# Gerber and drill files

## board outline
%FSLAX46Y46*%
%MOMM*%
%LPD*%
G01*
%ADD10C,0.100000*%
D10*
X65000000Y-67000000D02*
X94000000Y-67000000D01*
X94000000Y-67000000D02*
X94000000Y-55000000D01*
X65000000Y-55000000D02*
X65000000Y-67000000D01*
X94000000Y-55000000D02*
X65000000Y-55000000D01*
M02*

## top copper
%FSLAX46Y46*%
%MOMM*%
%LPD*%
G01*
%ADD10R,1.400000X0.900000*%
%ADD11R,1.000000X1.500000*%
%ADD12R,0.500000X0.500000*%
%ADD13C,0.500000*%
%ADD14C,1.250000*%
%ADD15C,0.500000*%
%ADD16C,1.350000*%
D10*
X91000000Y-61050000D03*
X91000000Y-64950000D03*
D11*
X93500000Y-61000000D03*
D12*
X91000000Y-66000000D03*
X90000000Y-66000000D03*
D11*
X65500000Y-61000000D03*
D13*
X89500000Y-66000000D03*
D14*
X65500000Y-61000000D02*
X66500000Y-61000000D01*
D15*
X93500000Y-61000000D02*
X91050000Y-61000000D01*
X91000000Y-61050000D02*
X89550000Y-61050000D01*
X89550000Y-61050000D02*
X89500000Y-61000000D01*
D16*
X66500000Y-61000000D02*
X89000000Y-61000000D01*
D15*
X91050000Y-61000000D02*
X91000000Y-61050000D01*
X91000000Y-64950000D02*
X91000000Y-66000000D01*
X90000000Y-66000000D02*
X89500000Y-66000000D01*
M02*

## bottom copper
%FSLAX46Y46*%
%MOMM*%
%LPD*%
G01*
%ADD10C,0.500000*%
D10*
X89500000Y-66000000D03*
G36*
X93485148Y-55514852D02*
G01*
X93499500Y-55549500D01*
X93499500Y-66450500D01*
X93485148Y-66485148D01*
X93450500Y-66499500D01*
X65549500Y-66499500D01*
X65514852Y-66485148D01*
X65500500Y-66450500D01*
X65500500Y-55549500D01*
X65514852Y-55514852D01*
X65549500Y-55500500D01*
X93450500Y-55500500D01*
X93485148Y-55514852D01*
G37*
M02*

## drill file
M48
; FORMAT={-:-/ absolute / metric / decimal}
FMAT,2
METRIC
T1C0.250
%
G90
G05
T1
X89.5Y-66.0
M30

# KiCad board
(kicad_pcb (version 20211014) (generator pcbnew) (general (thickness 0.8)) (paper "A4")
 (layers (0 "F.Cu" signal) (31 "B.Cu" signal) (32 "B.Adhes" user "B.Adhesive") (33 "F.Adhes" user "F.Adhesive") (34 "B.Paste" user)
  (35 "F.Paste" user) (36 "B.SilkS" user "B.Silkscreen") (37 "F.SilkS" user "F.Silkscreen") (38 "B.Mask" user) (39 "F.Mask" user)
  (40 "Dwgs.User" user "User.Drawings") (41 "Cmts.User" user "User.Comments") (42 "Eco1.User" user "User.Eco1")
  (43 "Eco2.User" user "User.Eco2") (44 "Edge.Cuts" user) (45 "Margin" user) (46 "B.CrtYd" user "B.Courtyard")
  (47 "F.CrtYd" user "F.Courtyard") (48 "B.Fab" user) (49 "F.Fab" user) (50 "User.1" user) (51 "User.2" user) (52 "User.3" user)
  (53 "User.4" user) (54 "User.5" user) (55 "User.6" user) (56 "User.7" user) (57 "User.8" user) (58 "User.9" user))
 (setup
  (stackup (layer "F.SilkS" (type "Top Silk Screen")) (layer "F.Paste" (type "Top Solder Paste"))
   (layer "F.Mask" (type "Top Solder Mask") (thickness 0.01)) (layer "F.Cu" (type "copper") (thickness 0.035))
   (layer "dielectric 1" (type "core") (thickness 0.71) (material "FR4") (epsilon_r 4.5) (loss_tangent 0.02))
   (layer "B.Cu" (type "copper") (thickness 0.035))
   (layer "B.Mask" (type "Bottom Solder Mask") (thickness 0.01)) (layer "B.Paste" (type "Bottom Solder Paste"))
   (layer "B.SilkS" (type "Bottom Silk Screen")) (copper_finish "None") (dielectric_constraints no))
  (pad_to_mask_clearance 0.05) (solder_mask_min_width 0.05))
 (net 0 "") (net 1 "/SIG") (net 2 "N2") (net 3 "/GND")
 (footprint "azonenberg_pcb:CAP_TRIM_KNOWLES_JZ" (layer "F.Cu") (at 91 63 -90)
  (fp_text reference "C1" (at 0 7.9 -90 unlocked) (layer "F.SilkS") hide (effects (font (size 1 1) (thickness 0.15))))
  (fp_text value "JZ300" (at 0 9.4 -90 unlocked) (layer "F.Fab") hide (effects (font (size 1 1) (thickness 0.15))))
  (pad "1" smd rect (at -1.95 0 270) (size 0.9 1.4) (layers "F.Cu" "F.Paste" "F.Mask") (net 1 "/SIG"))
  (pad "2" smd rect (at 1.95 0 270) (size 0.9 1.4) (layers "F.Cu" "F.Paste" "F.Mask") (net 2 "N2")))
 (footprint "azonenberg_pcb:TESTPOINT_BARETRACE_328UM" (layer "F.Cu") (at 93.5 61 90) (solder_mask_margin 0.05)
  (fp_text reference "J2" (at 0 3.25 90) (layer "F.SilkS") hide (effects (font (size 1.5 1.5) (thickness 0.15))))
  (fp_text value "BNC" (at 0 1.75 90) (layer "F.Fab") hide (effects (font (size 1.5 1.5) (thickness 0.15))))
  (pad "1" smd rect locked (at 0 0 90) (size 1.5 1) (layers "F.Cu" "F.Mask") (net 1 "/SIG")))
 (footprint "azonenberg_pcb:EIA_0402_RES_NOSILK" (layer "F.Cu") (at 90.5 66 180)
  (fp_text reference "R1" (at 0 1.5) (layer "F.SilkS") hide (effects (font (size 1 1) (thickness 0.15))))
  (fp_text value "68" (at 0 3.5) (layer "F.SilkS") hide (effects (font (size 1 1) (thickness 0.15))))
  (pad "1" smd rect (at -0.5 0 180) (size 0.5 0.5) (layers "F.Cu" "F.Paste" "F.Mask") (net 2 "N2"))
  (pad "2" smd rect (at 0.5 0 180) (size 0.5 0.5) (layers "F.Cu" "F.Paste" "F.Mask") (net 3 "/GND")))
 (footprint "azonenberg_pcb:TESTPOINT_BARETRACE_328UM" (layer "F.Cu") (at 65.5 61 90) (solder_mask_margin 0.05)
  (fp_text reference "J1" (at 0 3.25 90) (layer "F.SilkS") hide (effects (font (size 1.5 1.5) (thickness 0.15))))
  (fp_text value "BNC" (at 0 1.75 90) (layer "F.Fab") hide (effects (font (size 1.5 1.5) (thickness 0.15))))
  (pad "1" smd rect locked (at 0 0 90) (size 1.5 1) (layers "F.Cu" "F.Mask") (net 1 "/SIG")))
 (gr_line (start 65 67) (end 94 67) (layer "Edge.Cuts") (width 0.1))
 (gr_line (start 94 67) (end 94 55) (layer "Edge.Cuts") (width 0.1))
 (gr_line (start 65 55) (end 65 67) (layer "Edge.Cuts") (width 0.1))
 (gr_line (start 94 55) (end 65 55) (layer "Edge.Cuts") (width 0.1))
 (segment (start 65.5 61) (end 66.5 61) (width 1.25) (layer "F.Cu") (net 1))
 (segment (start 93.5 61) (end 91.05 61) (width 0.5) (layer "F.Cu") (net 1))
 (segment (start 91 61.05) (end 89.55 61.05) (width 0.5) (layer "F.Cu") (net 1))
 (segment (start 89.55 61.05) (end 89.5 61) (width 0.5) (layer "F.Cu") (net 1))
 (segment (start 66.5 61) (end 89 61) (width 1.35) (layer "F.Cu") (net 1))
 (segment (start 91.05 61) (end 91 61.05) (width 0.5) (layer "F.Cu") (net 1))
 (segment (start 91 64.95) (end 91 66) (width 0.5) (layer "F.Cu") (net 2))
 (segment (start 90 66) (end 89.5 66) (width 0.5) (layer "F.Cu") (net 3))
 (via (at 89.5 66) (size 0.5) (drill 0.25) (layers "F.Cu" "B.Cu") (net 3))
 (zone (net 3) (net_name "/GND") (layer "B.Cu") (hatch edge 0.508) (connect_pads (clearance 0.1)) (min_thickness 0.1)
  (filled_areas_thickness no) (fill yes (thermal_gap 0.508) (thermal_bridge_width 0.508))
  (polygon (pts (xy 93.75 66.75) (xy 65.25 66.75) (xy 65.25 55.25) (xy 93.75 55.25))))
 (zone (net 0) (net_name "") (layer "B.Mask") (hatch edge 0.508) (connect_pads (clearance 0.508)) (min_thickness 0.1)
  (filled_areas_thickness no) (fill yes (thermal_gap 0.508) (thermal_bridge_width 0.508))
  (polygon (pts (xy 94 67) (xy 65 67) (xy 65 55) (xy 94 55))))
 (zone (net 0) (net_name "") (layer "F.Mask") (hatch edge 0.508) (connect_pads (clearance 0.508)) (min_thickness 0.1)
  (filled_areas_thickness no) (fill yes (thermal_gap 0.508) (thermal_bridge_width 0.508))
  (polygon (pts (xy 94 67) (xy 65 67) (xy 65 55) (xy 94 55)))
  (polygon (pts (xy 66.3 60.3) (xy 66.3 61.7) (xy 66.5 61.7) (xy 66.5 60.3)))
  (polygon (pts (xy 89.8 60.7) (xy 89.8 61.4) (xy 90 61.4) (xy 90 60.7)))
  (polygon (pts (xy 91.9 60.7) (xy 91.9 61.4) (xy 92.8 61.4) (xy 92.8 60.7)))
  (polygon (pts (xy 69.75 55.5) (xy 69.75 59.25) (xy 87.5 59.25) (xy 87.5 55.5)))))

